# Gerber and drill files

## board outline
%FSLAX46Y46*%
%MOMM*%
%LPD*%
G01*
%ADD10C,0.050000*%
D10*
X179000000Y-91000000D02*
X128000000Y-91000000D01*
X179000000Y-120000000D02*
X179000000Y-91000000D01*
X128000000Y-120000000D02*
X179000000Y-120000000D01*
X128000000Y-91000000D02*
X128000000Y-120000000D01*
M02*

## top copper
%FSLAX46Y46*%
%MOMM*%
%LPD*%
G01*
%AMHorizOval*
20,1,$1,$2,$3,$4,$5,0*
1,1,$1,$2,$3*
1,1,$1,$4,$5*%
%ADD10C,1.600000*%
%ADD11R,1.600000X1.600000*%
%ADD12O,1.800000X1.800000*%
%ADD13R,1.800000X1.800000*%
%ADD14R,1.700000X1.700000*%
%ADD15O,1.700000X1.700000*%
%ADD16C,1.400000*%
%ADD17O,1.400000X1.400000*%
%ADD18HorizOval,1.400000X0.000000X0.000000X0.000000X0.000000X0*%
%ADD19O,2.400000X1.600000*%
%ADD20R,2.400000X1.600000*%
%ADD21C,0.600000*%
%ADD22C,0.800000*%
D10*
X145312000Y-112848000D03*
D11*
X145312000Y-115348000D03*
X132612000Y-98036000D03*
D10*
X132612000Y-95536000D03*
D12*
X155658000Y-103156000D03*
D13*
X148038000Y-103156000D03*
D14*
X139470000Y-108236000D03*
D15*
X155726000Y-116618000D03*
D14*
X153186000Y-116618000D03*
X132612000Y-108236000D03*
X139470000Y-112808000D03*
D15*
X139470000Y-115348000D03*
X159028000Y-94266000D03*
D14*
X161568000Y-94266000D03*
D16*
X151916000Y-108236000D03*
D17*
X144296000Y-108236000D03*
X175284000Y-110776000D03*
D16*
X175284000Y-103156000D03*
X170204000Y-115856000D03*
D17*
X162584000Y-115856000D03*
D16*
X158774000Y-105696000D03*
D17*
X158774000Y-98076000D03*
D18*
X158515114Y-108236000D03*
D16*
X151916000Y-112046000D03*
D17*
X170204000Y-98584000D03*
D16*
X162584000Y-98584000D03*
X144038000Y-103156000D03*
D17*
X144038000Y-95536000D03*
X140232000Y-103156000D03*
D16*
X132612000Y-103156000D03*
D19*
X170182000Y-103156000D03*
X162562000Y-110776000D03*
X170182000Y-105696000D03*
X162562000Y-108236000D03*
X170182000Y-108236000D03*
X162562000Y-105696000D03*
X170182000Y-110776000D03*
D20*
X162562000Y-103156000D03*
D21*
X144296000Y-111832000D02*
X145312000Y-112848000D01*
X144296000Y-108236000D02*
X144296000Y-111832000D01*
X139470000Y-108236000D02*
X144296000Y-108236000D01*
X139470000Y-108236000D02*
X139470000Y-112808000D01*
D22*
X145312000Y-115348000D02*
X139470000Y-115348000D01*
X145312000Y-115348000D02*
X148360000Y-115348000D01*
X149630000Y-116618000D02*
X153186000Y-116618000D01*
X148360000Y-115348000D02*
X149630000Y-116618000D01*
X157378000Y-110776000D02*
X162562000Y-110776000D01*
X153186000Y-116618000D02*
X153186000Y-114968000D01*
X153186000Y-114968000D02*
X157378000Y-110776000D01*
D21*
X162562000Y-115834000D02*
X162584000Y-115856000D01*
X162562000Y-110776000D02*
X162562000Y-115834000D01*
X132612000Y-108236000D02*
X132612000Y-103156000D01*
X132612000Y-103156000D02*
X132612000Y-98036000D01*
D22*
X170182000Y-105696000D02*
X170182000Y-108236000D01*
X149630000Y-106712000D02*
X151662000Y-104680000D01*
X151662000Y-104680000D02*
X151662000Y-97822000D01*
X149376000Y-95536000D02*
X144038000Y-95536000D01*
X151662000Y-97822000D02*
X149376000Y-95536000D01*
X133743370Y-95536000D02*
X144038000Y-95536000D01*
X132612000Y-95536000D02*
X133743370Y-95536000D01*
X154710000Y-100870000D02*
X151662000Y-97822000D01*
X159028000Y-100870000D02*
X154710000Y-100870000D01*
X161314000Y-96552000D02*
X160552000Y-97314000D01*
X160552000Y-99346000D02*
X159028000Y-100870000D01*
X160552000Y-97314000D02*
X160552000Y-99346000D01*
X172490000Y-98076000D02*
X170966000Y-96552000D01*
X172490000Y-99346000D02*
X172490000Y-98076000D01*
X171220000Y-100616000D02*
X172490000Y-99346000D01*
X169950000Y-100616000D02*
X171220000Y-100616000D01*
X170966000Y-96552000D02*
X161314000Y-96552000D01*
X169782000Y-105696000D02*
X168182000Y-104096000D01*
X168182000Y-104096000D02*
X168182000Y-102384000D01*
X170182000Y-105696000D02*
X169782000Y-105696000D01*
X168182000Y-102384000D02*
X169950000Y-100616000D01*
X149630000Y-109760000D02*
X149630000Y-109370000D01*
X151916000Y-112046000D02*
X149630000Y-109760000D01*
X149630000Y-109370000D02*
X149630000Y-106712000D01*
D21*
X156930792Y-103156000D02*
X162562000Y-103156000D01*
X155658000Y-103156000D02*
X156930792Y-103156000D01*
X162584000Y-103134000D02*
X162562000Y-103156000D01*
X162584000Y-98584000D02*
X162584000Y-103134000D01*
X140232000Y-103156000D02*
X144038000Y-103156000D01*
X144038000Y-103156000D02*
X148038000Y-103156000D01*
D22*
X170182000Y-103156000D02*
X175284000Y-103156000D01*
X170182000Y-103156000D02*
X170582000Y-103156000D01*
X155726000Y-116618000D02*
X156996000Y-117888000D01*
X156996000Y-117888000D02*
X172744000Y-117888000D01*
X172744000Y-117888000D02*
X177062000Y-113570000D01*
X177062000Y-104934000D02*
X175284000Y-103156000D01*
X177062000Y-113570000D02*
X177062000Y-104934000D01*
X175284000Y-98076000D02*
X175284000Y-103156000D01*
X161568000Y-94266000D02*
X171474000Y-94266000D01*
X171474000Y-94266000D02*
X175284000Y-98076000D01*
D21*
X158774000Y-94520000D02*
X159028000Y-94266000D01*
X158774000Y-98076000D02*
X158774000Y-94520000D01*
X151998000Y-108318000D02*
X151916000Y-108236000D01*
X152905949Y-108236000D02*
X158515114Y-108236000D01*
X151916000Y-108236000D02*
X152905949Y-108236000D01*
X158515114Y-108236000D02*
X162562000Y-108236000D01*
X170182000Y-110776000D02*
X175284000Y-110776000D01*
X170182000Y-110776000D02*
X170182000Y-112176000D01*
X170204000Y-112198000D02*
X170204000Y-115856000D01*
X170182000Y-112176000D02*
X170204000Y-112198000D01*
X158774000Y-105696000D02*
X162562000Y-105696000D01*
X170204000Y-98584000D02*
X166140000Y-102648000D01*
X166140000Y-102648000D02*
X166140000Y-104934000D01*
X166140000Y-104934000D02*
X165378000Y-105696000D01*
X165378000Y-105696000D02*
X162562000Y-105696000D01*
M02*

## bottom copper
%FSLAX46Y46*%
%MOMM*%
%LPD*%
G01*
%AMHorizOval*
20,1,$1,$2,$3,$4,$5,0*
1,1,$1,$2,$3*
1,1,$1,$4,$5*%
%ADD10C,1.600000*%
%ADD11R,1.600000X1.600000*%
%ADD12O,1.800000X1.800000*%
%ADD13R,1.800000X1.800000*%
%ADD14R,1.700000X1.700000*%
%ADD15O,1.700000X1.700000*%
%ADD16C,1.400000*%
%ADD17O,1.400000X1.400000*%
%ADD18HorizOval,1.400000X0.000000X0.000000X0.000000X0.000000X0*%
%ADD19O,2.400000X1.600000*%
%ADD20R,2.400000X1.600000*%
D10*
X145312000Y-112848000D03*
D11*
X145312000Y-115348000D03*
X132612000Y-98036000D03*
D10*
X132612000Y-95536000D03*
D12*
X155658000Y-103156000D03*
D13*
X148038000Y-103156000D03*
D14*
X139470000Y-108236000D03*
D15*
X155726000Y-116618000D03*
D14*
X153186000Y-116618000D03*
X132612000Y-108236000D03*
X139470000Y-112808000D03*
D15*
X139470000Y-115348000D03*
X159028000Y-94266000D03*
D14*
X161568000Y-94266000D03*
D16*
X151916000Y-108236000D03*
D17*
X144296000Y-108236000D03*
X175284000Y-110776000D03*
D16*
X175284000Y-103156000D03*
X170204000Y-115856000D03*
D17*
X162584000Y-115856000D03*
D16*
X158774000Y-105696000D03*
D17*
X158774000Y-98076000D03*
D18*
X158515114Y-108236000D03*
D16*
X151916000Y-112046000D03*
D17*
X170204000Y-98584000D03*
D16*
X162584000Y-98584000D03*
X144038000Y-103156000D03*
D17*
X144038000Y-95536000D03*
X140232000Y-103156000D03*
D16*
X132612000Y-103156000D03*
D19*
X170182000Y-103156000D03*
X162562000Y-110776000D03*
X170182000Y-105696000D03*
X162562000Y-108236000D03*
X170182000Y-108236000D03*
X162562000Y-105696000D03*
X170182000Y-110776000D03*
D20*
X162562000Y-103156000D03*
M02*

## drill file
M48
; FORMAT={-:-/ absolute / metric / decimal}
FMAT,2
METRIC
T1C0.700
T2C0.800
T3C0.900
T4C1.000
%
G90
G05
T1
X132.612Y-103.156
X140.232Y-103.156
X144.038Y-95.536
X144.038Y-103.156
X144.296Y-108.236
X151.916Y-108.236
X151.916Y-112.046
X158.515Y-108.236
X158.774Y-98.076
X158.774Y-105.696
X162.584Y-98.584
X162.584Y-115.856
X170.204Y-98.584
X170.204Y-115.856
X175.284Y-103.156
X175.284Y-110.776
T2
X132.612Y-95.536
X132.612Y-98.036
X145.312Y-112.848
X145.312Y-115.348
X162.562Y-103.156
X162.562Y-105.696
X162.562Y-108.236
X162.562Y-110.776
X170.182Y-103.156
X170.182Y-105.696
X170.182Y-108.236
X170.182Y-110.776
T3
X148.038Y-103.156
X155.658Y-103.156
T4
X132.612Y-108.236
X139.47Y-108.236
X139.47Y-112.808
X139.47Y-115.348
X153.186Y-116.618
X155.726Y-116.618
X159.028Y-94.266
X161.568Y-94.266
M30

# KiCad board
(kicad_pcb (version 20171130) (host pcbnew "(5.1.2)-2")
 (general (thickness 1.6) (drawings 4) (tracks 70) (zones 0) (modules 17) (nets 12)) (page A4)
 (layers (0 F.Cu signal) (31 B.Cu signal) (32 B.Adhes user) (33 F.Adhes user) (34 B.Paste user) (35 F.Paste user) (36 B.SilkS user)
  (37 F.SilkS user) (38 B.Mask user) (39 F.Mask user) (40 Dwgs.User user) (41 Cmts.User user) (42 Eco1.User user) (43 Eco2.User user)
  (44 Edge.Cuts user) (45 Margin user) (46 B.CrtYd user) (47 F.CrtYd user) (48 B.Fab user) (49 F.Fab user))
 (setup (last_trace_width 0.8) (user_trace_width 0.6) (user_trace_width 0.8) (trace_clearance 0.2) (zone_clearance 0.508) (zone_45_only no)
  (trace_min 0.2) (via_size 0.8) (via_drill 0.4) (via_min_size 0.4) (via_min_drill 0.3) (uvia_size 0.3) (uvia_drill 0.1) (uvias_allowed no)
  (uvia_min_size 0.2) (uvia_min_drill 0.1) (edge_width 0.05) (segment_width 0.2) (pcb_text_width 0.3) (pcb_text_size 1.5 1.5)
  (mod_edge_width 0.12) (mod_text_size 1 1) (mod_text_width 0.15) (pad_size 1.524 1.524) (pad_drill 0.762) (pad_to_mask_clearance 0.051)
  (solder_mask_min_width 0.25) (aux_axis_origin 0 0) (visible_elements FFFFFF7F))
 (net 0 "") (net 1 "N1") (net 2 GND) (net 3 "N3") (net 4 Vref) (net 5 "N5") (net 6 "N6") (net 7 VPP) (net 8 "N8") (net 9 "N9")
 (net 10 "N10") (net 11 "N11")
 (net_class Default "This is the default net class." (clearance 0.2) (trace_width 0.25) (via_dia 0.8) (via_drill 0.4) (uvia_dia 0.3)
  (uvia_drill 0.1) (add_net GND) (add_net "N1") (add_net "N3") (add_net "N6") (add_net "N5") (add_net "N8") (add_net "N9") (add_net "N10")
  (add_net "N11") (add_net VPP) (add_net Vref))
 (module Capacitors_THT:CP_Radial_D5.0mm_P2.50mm (layer F.Cu) (at 145.312 115.348 90)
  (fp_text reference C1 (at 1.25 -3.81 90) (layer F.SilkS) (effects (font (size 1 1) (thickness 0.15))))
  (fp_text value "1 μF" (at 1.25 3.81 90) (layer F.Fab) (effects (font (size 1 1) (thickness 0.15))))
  (pad 2 thru_hole circle (at 2.5 0 90) (size 1.6 1.6) (drill 0.8) (layers *.Cu *.Mask) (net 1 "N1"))
  (pad 1 thru_hole rect (at 0 0 90) (size 1.6 1.6) (drill 0.8) (layers *.Cu *.Mask) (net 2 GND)))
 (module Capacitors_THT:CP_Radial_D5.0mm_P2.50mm (layer F.Cu) (at 132.612 98.036 90)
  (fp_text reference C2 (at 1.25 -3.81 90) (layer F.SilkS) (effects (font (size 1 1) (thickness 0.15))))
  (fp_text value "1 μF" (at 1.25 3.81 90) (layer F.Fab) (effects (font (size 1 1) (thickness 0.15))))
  (pad 1 thru_hole rect (at 0 0 90) (size 1.6 1.6) (drill 0.8) (layers *.Cu *.Mask) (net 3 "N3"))
  (pad 2 thru_hole circle (at 2.5 0 90) (size 1.6 1.6) (drill 0.8) (layers *.Cu *.Mask) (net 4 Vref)))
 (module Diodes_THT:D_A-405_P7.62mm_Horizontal (layer F.Cu) (at 148.038 103.156)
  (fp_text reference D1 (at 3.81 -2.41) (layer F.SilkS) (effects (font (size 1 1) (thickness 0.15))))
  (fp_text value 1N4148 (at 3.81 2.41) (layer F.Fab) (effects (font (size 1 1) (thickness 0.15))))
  (pad 2 thru_hole oval (at 7.62 0) (size 1.8 1.8) (drill 0.9) (layers *.Cu *.Mask) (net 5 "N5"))
  (pad 1 thru_hole rect (at 0 0) (size 1.8 1.8) (drill 0.9) (layers *.Cu *.Mask) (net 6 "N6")))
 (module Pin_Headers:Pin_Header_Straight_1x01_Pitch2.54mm (layer F.Cu) (at 139.47 108.236 90)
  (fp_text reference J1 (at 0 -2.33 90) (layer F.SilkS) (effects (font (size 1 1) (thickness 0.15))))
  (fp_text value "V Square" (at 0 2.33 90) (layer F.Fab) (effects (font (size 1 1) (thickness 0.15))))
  (pad 1 thru_hole rect (at 0 0 90) (size 1.7 1.7) (drill 1) (layers *.Cu *.Mask) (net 1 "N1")))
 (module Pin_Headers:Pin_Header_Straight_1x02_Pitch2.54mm (layer F.Cu) (at 153.186 116.618 90)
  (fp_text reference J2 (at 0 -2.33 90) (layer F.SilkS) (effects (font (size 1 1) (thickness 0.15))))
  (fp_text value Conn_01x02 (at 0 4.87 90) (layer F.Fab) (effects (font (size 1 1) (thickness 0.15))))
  (pad 2 thru_hole oval (at 0 2.54 90) (size 1.7 1.7) (drill 1) (layers *.Cu *.Mask) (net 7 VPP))
  (pad 1 thru_hole rect (at 0 0 90) (size 1.7 1.7) (drill 1) (layers *.Cu *.Mask) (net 2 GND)))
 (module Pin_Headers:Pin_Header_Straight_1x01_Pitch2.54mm (layer F.Cu) (at 132.612 108.236 90)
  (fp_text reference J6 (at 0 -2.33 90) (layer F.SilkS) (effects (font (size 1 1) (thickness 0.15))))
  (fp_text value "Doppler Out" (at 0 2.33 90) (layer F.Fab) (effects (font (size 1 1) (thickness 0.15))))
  (pad 1 thru_hole rect (at 0 0 90) (size 1.7 1.7) (drill 1) (layers *.Cu *.Mask) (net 3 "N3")))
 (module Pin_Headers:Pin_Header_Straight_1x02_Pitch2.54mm (layer F.Cu) (at 139.47 112.808)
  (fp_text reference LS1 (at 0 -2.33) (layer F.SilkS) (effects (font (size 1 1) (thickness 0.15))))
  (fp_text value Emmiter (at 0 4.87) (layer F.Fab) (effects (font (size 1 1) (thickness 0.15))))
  (pad 1 thru_hole rect (at 0 0) (size 1.7 1.7) (drill 1) (layers *.Cu *.Mask) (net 1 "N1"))
  (pad 2 thru_hole oval (at 0 2.54) (size 1.7 1.7) (drill 1) (layers *.Cu *.Mask) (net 2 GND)))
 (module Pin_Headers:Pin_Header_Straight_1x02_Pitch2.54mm (layer F.Cu) (at 161.568 94.266 270)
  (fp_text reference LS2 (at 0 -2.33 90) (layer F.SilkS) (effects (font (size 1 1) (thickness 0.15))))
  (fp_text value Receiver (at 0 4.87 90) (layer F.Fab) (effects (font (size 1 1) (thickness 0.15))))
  (pad 2 thru_hole oval (at 0 2.54 270) (size 1.7 1.7) (drill 1) (layers *.Cu *.Mask) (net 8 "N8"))
  (pad 1 thru_hole rect (at 0 0 270) (size 1.7 1.7) (drill 1) (layers *.Cu *.Mask) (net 7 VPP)))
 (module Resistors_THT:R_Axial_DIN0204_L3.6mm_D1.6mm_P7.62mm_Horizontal (layer F.Cu) (at 151.916 108.236 180)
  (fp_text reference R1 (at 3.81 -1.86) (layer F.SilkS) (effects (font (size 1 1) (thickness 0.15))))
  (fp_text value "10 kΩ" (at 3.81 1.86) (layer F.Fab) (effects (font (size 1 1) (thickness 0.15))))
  (pad 1 thru_hole circle (at 0 0 180) (size 1.4 1.4) (drill 0.7) (layers *.Cu *.Mask) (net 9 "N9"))
  (pad 2 thru_hole oval (at 7.62 0 180) (size 1.4 1.4) (drill 0.7) (layers *.Cu *.Mask) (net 1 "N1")))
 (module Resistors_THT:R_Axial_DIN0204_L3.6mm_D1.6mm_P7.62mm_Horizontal (layer F.Cu) (at 175.284 103.156 270)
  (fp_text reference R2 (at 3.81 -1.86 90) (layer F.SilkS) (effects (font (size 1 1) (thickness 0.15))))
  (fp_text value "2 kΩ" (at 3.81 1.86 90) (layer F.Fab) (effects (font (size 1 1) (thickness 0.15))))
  (pad 2 thru_hole oval (at 7.62 0 270) (size 1.4 1.4) (drill 0.7) (layers *.Cu *.Mask) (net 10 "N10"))
  (pad 1 thru_hole circle (at 0 0 270) (size 1.4 1.4) (drill 0.7) (layers *.Cu *.Mask) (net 7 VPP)))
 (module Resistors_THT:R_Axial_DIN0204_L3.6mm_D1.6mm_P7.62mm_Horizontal (layer F.Cu) (at 170.204 115.856 180)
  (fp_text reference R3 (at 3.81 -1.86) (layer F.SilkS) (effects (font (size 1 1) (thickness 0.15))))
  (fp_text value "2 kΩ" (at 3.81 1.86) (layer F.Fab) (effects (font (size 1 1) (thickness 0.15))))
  (pad 1 thru_hole circle (at 0 0 180) (size 1.4 1.4) (drill 0.7) (layers *.Cu *.Mask) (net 10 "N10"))
  (pad 2 thru_hole oval (at 7.62 0 180) (size 1.4 1.4) (drill 0.7) (layers *.Cu *.Mask) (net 2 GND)))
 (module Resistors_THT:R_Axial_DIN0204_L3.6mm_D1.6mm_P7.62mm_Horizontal (layer F.Cu) (at 158.774 105.696 90)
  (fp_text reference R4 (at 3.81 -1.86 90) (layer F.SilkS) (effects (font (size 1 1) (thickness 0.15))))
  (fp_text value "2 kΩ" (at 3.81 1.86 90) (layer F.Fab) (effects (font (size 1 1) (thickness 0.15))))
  (pad 1 thru_hole circle (at 0 0 90) (size 1.4 1.4) (drill 0.7) (layers *.Cu *.Mask) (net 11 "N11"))
  (pad 2 thru_hole oval (at 7.62 0 90) (size 1.4 1.4) (drill 0.7) (layers *.Cu *.Mask) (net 8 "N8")))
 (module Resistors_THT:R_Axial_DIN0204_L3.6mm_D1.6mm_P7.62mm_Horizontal (layer F.Cu) (at 151.916 112.046 30)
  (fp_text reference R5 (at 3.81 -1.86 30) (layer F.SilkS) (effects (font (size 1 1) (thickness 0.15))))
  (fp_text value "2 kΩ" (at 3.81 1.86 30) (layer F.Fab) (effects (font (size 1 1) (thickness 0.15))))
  (pad 2 thru_hole oval (at 7.62 0 30) (size 1.4 1.4) (drill 0.7) (layers *.Cu *.Mask) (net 9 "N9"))
  (pad 1 thru_hole circle (at 0 0 30) (size 1.4 1.4) (drill 0.7) (layers *.Cu *.Mask) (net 4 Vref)))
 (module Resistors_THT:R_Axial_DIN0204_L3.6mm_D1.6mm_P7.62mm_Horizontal (layer F.Cu) (at 162.584 98.584)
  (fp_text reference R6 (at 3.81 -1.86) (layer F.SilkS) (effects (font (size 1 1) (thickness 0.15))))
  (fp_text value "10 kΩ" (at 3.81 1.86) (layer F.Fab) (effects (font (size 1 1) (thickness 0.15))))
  (pad 2 thru_hole oval (at 7.62 0) (size 1.4 1.4) (drill 0.7) (layers *.Cu *.Mask) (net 11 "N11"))
  (pad 1 thru_hole circle (at 0 0) (size 1.4 1.4) (drill 0.7) (layers *.Cu *.Mask) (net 5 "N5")))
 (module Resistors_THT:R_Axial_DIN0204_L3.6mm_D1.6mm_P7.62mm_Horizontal (layer F.Cu) (at 144.038 103.156 90)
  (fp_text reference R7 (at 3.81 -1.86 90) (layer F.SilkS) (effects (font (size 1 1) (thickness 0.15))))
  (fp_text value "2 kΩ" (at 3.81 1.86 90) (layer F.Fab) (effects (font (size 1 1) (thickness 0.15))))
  (pad 1 thru_hole circle (at 0 0 90) (size 1.4 1.4) (drill 0.7) (layers *.Cu *.Mask) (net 6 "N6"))
  (pad 2 thru_hole oval (at 7.62 0 90) (size 1.4 1.4) (drill 0.7) (layers *.Cu *.Mask) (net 4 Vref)))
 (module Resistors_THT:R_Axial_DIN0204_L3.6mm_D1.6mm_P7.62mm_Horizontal (layer F.Cu) (at 132.612 103.156)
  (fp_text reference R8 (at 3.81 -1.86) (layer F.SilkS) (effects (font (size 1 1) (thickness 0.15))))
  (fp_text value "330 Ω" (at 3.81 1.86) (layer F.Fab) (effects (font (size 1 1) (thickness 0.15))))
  (pad 2 thru_hole oval (at 7.62 0) (size 1.4 1.4) (drill 0.7) (layers *.Cu *.Mask) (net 6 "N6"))
  (pad 1 thru_hole circle (at 0 0) (size 1.4 1.4) (drill 0.7) (layers *.Cu *.Mask) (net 3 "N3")))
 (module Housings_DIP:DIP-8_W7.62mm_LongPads (layer F.Cu) (at 162.562 103.156)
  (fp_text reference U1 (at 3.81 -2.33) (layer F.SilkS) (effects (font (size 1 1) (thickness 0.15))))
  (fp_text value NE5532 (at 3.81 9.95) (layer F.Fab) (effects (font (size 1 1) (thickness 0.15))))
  (pad 8 thru_hole oval (at 7.62 0) (size 2.4 1.6) (drill 0.8) (layers *.Cu *.Mask) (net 7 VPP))
  (pad 4 thru_hole oval (at 0 7.62) (size 2.4 1.6) (drill 0.8) (layers *.Cu *.Mask) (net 2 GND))
  (pad 7 thru_hole oval (at 7.62 2.54) (size 2.4 1.6) (drill 0.8) (layers *.Cu *.Mask) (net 4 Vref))
  (pad 3 thru_hole oval (at 0 5.08) (size 2.4 1.6) (drill 0.8) (layers *.Cu *.Mask) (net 9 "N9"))
  (pad 6 thru_hole oval (at 7.62 5.08) (size 2.4 1.6) (drill 0.8) (layers *.Cu *.Mask) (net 4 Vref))
  (pad 2 thru_hole oval (at 0 2.54) (size 2.4 1.6) (drill 0.8) (layers *.Cu *.Mask) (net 11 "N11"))
  (pad 5 thru_hole oval (at 7.62 7.62) (size 2.4 1.6) (drill 0.8) (layers *.Cu *.Mask) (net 10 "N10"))
  (pad 1 thru_hole rect (at 0 0) (size 2.4 1.6) (drill 0.8) (layers *.Cu *.Mask) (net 5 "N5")))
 (gr_line (start 179 91) (end 128 91) (layer Edge.Cuts) (width 0.05))
 (gr_line (start 179 120) (end 179 91) (layer Edge.Cuts) (width 0.05))
 (gr_line (start 128 120) (end 179 120) (layer Edge.Cuts) (width 0.05))
 (gr_line (start 128 91) (end 128 120) (layer Edge.Cuts) (width 0.05))
 (segment (start 144.296 111.832) (end 145.312 112.848) (width 0.6) (layer F.Cu) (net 1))
 (segment (start 144.296 108.236) (end 144.296 111.832) (width 0.6) (layer F.Cu) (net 1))
 (segment (start 139.47 108.236) (end 144.296 108.236) (width 0.6) (layer F.Cu) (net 1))
 (segment (start 139.47 108.236) (end 139.47 112.808) (width 0.6) (layer F.Cu) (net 1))
 (segment (start 145.312 115.348) (end 139.47 115.348) (width 0.8) (layer F.Cu) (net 2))
 (segment (start 145.312 115.348) (end 148.36 115.348) (width 0.8) (layer F.Cu) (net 2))
 (segment (start 149.63 116.618) (end 153.186 116.618) (width 0.8) (layer F.Cu) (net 2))
 (segment (start 148.36 115.348) (end 149.63 116.618) (width 0.8) (layer F.Cu) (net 2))
 (segment (start 157.378 110.776) (end 162.562 110.776) (width 0.8) (layer F.Cu) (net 2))
 (segment (start 153.186 116.618) (end 153.186 114.968) (width 0.8) (layer F.Cu) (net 2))
 (segment (start 153.186 114.968) (end 157.378 110.776) (width 0.8) (layer F.Cu) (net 2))
 (segment (start 162.562 115.834) (end 162.584 115.856) (width 0.6) (layer F.Cu) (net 2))
 (segment (start 162.562 110.776) (end 162.562 115.834) (width 0.6) (layer F.Cu) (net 2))
 (segment (start 132.612 108.236) (end 132.612 103.156) (width 0.6) (layer F.Cu) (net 3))
 (segment (start 132.612 103.156) (end 132.612 98.036) (width 0.6) (layer F.Cu) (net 3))
 (segment (start 170.182 105.696) (end 170.182 108.236) (width 0.8) (layer F.Cu) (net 4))
 (segment (start 149.63 106.712) (end 151.662 104.68) (width 0.8) (layer F.Cu) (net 4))
 (segment (start 151.662 104.68) (end 151.662 97.822) (width 0.8) (layer F.Cu) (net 4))
 (segment (start 149.376 95.536) (end 144.038 95.536) (width 0.8) (layer F.Cu) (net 4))
 (segment (start 151.662 97.822) (end 149.376 95.536) (width 0.8) (layer F.Cu) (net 4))
 (segment (start 133.74337 95.536) (end 144.038 95.536) (width 0.8) (layer F.Cu) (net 4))
 (segment (start 132.612 95.536) (end 133.74337 95.536) (width 0.8) (layer F.Cu) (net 4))
 (segment (start 154.71 100.87) (end 151.662 97.822) (width 0.8) (layer F.Cu) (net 4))
 (segment (start 159.028 100.87) (end 154.71 100.87) (width 0.8) (layer F.Cu) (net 4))
 (segment (start 161.314 96.552) (end 160.552 97.314) (width 0.8) (layer F.Cu) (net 4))
 (segment (start 160.552 99.346) (end 159.028 100.87) (width 0.8) (layer F.Cu) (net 4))
 (segment (start 160.552 97.314) (end 160.552 99.346) (width 0.8) (layer F.Cu) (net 4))
 (segment (start 172.49 98.076) (end 170.966 96.552) (width 0.8) (layer F.Cu) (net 4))
 (segment (start 172.49 99.346) (end 172.49 98.076) (width 0.8) (layer F.Cu) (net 4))
 (segment (start 171.22 100.616) (end 172.49 99.346) (width 0.8) (layer F.Cu) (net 4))
 (segment (start 169.95 100.616) (end 171.22 100.616) (width 0.8) (layer F.Cu) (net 4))
 (segment (start 170.966 96.552) (end 161.314 96.552) (width 0.8) (layer F.Cu) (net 4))
 (segment (start 169.782 105.696) (end 168.182 104.096) (width 0.8) (layer F.Cu) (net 4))
 (segment (start 168.182 104.096) (end 168.182 102.384) (width 0.8) (layer F.Cu) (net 4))
 (segment (start 170.182 105.696) (end 169.782 105.696) (width 0.8) (layer F.Cu) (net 4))
 (segment (start 168.182 102.384) (end 169.95 100.616) (width 0.8) (layer F.Cu) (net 4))
 (segment (start 149.63 109.76) (end 149.63 109.37) (width 0.8) (layer F.Cu) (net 4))
 (segment (start 151.916 112.046) (end 149.63 109.76) (width 0.8) (layer F.Cu) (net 4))
 (segment (start 149.63 109.37) (end 149.63 106.712) (width 0.8) (layer F.Cu) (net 4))
 (segment (start 156.930792 103.156) (end 162.562 103.156) (width 0.6) (layer F.Cu) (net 5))
 (segment (start 155.658 103.156) (end 156.930792 103.156) (width 0.6) (layer F.Cu) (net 5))
 (segment (start 162.584 103.134) (end 162.562 103.156) (width 0.6) (layer F.Cu) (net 5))
 (segment (start 162.584 98.584) (end 162.584 103.134) (width 0.6) (layer F.Cu) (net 5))
 (segment (start 140.232 103.156) (end 144.038 103.156) (width 0.6) (layer F.Cu) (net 6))
 (segment (start 144.038 103.156) (end 148.038 103.156) (width 0.6) (layer F.Cu) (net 6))
 (segment (start 170.182 103.156) (end 175.284 103.156) (width 0.8) (layer F.Cu) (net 7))
 (segment (start 170.182 103.156) (end 170.582 103.156) (width 0.8) (layer F.Cu) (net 7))
 (segment (start 155.726 116.618) (end 156.996 117.888) (width 0.8) (layer F.Cu) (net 7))
 (segment (start 156.996 117.888) (end 172.744 117.888) (width 0.8) (layer F.Cu) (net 7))
 (segment (start 172.744 117.888) (end 177.062 113.57) (width 0.8) (layer F.Cu) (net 7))
 (segment (start 177.062 104.934) (end 175.284 103.156) (width 0.8) (layer F.Cu) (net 7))
 (segment (start 177.062 113.57) (end 177.062 104.934) (width 0.8) (layer F.Cu) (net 7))
 (segment (start 175.284 98.076) (end 175.284 103.156) (width 0.8) (layer F.Cu) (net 7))
 (segment (start 161.568 94.266) (end 171.474 94.266) (width 0.8) (layer F.Cu) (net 7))
 (segment (start 171.474 94.266) (end 175.284 98.076) (width 0.8) (layer F.Cu) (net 7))
 (segment (start 158.774 94.52) (end 159.028 94.266) (width 0.6) (layer F.Cu) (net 8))
 (segment (start 158.774 98.076) (end 158.774 94.52) (width 0.6) (layer F.Cu) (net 8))
 (segment (start 151.998 108.318) (end 151.916 108.236) (width 0.6) (layer F.Cu) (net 9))
 (segment (start 152.905949 108.236) (end 158.515114 108.236) (width 0.6) (layer F.Cu) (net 9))
 (segment (start 151.916 108.236) (end 152.905949 108.236) (width 0.6) (layer F.Cu) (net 9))
 (segment (start 158.515114 108.236) (end 162.562 108.236) (width 0.6) (layer F.Cu) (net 9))
 (segment (start 170.182 110.776) (end 175.284 110.776) (width 0.6) (layer F.Cu) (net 10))
 (segment (start 170.182 110.776) (end 170.182 112.176) (width 0.6) (layer F.Cu) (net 10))
 (segment (start 170.204 112.198) (end 170.204 115.856) (width 0.6) (layer F.Cu) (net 10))
 (segment (start 170.182 112.176) (end 170.204 112.198) (width 0.6) (layer F.Cu) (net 10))
 (segment (start 158.774 105.696) (end 162.562 105.696) (width 0.6) (layer F.Cu) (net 11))
 (segment (start 170.204 98.584) (end 166.14 102.648) (width 0.6) (layer F.Cu) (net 11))
 (segment (start 166.14 102.648) (end 166.14 104.934) (width 0.6) (layer F.Cu) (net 11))
 (segment (start 166.14 104.934) (end 165.378 105.696) (width 0.6) (layer F.Cu) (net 11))
 (segment (start 165.378 105.696) (end 162.562 105.696) (width 0.6) (layer F.Cu) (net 11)))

